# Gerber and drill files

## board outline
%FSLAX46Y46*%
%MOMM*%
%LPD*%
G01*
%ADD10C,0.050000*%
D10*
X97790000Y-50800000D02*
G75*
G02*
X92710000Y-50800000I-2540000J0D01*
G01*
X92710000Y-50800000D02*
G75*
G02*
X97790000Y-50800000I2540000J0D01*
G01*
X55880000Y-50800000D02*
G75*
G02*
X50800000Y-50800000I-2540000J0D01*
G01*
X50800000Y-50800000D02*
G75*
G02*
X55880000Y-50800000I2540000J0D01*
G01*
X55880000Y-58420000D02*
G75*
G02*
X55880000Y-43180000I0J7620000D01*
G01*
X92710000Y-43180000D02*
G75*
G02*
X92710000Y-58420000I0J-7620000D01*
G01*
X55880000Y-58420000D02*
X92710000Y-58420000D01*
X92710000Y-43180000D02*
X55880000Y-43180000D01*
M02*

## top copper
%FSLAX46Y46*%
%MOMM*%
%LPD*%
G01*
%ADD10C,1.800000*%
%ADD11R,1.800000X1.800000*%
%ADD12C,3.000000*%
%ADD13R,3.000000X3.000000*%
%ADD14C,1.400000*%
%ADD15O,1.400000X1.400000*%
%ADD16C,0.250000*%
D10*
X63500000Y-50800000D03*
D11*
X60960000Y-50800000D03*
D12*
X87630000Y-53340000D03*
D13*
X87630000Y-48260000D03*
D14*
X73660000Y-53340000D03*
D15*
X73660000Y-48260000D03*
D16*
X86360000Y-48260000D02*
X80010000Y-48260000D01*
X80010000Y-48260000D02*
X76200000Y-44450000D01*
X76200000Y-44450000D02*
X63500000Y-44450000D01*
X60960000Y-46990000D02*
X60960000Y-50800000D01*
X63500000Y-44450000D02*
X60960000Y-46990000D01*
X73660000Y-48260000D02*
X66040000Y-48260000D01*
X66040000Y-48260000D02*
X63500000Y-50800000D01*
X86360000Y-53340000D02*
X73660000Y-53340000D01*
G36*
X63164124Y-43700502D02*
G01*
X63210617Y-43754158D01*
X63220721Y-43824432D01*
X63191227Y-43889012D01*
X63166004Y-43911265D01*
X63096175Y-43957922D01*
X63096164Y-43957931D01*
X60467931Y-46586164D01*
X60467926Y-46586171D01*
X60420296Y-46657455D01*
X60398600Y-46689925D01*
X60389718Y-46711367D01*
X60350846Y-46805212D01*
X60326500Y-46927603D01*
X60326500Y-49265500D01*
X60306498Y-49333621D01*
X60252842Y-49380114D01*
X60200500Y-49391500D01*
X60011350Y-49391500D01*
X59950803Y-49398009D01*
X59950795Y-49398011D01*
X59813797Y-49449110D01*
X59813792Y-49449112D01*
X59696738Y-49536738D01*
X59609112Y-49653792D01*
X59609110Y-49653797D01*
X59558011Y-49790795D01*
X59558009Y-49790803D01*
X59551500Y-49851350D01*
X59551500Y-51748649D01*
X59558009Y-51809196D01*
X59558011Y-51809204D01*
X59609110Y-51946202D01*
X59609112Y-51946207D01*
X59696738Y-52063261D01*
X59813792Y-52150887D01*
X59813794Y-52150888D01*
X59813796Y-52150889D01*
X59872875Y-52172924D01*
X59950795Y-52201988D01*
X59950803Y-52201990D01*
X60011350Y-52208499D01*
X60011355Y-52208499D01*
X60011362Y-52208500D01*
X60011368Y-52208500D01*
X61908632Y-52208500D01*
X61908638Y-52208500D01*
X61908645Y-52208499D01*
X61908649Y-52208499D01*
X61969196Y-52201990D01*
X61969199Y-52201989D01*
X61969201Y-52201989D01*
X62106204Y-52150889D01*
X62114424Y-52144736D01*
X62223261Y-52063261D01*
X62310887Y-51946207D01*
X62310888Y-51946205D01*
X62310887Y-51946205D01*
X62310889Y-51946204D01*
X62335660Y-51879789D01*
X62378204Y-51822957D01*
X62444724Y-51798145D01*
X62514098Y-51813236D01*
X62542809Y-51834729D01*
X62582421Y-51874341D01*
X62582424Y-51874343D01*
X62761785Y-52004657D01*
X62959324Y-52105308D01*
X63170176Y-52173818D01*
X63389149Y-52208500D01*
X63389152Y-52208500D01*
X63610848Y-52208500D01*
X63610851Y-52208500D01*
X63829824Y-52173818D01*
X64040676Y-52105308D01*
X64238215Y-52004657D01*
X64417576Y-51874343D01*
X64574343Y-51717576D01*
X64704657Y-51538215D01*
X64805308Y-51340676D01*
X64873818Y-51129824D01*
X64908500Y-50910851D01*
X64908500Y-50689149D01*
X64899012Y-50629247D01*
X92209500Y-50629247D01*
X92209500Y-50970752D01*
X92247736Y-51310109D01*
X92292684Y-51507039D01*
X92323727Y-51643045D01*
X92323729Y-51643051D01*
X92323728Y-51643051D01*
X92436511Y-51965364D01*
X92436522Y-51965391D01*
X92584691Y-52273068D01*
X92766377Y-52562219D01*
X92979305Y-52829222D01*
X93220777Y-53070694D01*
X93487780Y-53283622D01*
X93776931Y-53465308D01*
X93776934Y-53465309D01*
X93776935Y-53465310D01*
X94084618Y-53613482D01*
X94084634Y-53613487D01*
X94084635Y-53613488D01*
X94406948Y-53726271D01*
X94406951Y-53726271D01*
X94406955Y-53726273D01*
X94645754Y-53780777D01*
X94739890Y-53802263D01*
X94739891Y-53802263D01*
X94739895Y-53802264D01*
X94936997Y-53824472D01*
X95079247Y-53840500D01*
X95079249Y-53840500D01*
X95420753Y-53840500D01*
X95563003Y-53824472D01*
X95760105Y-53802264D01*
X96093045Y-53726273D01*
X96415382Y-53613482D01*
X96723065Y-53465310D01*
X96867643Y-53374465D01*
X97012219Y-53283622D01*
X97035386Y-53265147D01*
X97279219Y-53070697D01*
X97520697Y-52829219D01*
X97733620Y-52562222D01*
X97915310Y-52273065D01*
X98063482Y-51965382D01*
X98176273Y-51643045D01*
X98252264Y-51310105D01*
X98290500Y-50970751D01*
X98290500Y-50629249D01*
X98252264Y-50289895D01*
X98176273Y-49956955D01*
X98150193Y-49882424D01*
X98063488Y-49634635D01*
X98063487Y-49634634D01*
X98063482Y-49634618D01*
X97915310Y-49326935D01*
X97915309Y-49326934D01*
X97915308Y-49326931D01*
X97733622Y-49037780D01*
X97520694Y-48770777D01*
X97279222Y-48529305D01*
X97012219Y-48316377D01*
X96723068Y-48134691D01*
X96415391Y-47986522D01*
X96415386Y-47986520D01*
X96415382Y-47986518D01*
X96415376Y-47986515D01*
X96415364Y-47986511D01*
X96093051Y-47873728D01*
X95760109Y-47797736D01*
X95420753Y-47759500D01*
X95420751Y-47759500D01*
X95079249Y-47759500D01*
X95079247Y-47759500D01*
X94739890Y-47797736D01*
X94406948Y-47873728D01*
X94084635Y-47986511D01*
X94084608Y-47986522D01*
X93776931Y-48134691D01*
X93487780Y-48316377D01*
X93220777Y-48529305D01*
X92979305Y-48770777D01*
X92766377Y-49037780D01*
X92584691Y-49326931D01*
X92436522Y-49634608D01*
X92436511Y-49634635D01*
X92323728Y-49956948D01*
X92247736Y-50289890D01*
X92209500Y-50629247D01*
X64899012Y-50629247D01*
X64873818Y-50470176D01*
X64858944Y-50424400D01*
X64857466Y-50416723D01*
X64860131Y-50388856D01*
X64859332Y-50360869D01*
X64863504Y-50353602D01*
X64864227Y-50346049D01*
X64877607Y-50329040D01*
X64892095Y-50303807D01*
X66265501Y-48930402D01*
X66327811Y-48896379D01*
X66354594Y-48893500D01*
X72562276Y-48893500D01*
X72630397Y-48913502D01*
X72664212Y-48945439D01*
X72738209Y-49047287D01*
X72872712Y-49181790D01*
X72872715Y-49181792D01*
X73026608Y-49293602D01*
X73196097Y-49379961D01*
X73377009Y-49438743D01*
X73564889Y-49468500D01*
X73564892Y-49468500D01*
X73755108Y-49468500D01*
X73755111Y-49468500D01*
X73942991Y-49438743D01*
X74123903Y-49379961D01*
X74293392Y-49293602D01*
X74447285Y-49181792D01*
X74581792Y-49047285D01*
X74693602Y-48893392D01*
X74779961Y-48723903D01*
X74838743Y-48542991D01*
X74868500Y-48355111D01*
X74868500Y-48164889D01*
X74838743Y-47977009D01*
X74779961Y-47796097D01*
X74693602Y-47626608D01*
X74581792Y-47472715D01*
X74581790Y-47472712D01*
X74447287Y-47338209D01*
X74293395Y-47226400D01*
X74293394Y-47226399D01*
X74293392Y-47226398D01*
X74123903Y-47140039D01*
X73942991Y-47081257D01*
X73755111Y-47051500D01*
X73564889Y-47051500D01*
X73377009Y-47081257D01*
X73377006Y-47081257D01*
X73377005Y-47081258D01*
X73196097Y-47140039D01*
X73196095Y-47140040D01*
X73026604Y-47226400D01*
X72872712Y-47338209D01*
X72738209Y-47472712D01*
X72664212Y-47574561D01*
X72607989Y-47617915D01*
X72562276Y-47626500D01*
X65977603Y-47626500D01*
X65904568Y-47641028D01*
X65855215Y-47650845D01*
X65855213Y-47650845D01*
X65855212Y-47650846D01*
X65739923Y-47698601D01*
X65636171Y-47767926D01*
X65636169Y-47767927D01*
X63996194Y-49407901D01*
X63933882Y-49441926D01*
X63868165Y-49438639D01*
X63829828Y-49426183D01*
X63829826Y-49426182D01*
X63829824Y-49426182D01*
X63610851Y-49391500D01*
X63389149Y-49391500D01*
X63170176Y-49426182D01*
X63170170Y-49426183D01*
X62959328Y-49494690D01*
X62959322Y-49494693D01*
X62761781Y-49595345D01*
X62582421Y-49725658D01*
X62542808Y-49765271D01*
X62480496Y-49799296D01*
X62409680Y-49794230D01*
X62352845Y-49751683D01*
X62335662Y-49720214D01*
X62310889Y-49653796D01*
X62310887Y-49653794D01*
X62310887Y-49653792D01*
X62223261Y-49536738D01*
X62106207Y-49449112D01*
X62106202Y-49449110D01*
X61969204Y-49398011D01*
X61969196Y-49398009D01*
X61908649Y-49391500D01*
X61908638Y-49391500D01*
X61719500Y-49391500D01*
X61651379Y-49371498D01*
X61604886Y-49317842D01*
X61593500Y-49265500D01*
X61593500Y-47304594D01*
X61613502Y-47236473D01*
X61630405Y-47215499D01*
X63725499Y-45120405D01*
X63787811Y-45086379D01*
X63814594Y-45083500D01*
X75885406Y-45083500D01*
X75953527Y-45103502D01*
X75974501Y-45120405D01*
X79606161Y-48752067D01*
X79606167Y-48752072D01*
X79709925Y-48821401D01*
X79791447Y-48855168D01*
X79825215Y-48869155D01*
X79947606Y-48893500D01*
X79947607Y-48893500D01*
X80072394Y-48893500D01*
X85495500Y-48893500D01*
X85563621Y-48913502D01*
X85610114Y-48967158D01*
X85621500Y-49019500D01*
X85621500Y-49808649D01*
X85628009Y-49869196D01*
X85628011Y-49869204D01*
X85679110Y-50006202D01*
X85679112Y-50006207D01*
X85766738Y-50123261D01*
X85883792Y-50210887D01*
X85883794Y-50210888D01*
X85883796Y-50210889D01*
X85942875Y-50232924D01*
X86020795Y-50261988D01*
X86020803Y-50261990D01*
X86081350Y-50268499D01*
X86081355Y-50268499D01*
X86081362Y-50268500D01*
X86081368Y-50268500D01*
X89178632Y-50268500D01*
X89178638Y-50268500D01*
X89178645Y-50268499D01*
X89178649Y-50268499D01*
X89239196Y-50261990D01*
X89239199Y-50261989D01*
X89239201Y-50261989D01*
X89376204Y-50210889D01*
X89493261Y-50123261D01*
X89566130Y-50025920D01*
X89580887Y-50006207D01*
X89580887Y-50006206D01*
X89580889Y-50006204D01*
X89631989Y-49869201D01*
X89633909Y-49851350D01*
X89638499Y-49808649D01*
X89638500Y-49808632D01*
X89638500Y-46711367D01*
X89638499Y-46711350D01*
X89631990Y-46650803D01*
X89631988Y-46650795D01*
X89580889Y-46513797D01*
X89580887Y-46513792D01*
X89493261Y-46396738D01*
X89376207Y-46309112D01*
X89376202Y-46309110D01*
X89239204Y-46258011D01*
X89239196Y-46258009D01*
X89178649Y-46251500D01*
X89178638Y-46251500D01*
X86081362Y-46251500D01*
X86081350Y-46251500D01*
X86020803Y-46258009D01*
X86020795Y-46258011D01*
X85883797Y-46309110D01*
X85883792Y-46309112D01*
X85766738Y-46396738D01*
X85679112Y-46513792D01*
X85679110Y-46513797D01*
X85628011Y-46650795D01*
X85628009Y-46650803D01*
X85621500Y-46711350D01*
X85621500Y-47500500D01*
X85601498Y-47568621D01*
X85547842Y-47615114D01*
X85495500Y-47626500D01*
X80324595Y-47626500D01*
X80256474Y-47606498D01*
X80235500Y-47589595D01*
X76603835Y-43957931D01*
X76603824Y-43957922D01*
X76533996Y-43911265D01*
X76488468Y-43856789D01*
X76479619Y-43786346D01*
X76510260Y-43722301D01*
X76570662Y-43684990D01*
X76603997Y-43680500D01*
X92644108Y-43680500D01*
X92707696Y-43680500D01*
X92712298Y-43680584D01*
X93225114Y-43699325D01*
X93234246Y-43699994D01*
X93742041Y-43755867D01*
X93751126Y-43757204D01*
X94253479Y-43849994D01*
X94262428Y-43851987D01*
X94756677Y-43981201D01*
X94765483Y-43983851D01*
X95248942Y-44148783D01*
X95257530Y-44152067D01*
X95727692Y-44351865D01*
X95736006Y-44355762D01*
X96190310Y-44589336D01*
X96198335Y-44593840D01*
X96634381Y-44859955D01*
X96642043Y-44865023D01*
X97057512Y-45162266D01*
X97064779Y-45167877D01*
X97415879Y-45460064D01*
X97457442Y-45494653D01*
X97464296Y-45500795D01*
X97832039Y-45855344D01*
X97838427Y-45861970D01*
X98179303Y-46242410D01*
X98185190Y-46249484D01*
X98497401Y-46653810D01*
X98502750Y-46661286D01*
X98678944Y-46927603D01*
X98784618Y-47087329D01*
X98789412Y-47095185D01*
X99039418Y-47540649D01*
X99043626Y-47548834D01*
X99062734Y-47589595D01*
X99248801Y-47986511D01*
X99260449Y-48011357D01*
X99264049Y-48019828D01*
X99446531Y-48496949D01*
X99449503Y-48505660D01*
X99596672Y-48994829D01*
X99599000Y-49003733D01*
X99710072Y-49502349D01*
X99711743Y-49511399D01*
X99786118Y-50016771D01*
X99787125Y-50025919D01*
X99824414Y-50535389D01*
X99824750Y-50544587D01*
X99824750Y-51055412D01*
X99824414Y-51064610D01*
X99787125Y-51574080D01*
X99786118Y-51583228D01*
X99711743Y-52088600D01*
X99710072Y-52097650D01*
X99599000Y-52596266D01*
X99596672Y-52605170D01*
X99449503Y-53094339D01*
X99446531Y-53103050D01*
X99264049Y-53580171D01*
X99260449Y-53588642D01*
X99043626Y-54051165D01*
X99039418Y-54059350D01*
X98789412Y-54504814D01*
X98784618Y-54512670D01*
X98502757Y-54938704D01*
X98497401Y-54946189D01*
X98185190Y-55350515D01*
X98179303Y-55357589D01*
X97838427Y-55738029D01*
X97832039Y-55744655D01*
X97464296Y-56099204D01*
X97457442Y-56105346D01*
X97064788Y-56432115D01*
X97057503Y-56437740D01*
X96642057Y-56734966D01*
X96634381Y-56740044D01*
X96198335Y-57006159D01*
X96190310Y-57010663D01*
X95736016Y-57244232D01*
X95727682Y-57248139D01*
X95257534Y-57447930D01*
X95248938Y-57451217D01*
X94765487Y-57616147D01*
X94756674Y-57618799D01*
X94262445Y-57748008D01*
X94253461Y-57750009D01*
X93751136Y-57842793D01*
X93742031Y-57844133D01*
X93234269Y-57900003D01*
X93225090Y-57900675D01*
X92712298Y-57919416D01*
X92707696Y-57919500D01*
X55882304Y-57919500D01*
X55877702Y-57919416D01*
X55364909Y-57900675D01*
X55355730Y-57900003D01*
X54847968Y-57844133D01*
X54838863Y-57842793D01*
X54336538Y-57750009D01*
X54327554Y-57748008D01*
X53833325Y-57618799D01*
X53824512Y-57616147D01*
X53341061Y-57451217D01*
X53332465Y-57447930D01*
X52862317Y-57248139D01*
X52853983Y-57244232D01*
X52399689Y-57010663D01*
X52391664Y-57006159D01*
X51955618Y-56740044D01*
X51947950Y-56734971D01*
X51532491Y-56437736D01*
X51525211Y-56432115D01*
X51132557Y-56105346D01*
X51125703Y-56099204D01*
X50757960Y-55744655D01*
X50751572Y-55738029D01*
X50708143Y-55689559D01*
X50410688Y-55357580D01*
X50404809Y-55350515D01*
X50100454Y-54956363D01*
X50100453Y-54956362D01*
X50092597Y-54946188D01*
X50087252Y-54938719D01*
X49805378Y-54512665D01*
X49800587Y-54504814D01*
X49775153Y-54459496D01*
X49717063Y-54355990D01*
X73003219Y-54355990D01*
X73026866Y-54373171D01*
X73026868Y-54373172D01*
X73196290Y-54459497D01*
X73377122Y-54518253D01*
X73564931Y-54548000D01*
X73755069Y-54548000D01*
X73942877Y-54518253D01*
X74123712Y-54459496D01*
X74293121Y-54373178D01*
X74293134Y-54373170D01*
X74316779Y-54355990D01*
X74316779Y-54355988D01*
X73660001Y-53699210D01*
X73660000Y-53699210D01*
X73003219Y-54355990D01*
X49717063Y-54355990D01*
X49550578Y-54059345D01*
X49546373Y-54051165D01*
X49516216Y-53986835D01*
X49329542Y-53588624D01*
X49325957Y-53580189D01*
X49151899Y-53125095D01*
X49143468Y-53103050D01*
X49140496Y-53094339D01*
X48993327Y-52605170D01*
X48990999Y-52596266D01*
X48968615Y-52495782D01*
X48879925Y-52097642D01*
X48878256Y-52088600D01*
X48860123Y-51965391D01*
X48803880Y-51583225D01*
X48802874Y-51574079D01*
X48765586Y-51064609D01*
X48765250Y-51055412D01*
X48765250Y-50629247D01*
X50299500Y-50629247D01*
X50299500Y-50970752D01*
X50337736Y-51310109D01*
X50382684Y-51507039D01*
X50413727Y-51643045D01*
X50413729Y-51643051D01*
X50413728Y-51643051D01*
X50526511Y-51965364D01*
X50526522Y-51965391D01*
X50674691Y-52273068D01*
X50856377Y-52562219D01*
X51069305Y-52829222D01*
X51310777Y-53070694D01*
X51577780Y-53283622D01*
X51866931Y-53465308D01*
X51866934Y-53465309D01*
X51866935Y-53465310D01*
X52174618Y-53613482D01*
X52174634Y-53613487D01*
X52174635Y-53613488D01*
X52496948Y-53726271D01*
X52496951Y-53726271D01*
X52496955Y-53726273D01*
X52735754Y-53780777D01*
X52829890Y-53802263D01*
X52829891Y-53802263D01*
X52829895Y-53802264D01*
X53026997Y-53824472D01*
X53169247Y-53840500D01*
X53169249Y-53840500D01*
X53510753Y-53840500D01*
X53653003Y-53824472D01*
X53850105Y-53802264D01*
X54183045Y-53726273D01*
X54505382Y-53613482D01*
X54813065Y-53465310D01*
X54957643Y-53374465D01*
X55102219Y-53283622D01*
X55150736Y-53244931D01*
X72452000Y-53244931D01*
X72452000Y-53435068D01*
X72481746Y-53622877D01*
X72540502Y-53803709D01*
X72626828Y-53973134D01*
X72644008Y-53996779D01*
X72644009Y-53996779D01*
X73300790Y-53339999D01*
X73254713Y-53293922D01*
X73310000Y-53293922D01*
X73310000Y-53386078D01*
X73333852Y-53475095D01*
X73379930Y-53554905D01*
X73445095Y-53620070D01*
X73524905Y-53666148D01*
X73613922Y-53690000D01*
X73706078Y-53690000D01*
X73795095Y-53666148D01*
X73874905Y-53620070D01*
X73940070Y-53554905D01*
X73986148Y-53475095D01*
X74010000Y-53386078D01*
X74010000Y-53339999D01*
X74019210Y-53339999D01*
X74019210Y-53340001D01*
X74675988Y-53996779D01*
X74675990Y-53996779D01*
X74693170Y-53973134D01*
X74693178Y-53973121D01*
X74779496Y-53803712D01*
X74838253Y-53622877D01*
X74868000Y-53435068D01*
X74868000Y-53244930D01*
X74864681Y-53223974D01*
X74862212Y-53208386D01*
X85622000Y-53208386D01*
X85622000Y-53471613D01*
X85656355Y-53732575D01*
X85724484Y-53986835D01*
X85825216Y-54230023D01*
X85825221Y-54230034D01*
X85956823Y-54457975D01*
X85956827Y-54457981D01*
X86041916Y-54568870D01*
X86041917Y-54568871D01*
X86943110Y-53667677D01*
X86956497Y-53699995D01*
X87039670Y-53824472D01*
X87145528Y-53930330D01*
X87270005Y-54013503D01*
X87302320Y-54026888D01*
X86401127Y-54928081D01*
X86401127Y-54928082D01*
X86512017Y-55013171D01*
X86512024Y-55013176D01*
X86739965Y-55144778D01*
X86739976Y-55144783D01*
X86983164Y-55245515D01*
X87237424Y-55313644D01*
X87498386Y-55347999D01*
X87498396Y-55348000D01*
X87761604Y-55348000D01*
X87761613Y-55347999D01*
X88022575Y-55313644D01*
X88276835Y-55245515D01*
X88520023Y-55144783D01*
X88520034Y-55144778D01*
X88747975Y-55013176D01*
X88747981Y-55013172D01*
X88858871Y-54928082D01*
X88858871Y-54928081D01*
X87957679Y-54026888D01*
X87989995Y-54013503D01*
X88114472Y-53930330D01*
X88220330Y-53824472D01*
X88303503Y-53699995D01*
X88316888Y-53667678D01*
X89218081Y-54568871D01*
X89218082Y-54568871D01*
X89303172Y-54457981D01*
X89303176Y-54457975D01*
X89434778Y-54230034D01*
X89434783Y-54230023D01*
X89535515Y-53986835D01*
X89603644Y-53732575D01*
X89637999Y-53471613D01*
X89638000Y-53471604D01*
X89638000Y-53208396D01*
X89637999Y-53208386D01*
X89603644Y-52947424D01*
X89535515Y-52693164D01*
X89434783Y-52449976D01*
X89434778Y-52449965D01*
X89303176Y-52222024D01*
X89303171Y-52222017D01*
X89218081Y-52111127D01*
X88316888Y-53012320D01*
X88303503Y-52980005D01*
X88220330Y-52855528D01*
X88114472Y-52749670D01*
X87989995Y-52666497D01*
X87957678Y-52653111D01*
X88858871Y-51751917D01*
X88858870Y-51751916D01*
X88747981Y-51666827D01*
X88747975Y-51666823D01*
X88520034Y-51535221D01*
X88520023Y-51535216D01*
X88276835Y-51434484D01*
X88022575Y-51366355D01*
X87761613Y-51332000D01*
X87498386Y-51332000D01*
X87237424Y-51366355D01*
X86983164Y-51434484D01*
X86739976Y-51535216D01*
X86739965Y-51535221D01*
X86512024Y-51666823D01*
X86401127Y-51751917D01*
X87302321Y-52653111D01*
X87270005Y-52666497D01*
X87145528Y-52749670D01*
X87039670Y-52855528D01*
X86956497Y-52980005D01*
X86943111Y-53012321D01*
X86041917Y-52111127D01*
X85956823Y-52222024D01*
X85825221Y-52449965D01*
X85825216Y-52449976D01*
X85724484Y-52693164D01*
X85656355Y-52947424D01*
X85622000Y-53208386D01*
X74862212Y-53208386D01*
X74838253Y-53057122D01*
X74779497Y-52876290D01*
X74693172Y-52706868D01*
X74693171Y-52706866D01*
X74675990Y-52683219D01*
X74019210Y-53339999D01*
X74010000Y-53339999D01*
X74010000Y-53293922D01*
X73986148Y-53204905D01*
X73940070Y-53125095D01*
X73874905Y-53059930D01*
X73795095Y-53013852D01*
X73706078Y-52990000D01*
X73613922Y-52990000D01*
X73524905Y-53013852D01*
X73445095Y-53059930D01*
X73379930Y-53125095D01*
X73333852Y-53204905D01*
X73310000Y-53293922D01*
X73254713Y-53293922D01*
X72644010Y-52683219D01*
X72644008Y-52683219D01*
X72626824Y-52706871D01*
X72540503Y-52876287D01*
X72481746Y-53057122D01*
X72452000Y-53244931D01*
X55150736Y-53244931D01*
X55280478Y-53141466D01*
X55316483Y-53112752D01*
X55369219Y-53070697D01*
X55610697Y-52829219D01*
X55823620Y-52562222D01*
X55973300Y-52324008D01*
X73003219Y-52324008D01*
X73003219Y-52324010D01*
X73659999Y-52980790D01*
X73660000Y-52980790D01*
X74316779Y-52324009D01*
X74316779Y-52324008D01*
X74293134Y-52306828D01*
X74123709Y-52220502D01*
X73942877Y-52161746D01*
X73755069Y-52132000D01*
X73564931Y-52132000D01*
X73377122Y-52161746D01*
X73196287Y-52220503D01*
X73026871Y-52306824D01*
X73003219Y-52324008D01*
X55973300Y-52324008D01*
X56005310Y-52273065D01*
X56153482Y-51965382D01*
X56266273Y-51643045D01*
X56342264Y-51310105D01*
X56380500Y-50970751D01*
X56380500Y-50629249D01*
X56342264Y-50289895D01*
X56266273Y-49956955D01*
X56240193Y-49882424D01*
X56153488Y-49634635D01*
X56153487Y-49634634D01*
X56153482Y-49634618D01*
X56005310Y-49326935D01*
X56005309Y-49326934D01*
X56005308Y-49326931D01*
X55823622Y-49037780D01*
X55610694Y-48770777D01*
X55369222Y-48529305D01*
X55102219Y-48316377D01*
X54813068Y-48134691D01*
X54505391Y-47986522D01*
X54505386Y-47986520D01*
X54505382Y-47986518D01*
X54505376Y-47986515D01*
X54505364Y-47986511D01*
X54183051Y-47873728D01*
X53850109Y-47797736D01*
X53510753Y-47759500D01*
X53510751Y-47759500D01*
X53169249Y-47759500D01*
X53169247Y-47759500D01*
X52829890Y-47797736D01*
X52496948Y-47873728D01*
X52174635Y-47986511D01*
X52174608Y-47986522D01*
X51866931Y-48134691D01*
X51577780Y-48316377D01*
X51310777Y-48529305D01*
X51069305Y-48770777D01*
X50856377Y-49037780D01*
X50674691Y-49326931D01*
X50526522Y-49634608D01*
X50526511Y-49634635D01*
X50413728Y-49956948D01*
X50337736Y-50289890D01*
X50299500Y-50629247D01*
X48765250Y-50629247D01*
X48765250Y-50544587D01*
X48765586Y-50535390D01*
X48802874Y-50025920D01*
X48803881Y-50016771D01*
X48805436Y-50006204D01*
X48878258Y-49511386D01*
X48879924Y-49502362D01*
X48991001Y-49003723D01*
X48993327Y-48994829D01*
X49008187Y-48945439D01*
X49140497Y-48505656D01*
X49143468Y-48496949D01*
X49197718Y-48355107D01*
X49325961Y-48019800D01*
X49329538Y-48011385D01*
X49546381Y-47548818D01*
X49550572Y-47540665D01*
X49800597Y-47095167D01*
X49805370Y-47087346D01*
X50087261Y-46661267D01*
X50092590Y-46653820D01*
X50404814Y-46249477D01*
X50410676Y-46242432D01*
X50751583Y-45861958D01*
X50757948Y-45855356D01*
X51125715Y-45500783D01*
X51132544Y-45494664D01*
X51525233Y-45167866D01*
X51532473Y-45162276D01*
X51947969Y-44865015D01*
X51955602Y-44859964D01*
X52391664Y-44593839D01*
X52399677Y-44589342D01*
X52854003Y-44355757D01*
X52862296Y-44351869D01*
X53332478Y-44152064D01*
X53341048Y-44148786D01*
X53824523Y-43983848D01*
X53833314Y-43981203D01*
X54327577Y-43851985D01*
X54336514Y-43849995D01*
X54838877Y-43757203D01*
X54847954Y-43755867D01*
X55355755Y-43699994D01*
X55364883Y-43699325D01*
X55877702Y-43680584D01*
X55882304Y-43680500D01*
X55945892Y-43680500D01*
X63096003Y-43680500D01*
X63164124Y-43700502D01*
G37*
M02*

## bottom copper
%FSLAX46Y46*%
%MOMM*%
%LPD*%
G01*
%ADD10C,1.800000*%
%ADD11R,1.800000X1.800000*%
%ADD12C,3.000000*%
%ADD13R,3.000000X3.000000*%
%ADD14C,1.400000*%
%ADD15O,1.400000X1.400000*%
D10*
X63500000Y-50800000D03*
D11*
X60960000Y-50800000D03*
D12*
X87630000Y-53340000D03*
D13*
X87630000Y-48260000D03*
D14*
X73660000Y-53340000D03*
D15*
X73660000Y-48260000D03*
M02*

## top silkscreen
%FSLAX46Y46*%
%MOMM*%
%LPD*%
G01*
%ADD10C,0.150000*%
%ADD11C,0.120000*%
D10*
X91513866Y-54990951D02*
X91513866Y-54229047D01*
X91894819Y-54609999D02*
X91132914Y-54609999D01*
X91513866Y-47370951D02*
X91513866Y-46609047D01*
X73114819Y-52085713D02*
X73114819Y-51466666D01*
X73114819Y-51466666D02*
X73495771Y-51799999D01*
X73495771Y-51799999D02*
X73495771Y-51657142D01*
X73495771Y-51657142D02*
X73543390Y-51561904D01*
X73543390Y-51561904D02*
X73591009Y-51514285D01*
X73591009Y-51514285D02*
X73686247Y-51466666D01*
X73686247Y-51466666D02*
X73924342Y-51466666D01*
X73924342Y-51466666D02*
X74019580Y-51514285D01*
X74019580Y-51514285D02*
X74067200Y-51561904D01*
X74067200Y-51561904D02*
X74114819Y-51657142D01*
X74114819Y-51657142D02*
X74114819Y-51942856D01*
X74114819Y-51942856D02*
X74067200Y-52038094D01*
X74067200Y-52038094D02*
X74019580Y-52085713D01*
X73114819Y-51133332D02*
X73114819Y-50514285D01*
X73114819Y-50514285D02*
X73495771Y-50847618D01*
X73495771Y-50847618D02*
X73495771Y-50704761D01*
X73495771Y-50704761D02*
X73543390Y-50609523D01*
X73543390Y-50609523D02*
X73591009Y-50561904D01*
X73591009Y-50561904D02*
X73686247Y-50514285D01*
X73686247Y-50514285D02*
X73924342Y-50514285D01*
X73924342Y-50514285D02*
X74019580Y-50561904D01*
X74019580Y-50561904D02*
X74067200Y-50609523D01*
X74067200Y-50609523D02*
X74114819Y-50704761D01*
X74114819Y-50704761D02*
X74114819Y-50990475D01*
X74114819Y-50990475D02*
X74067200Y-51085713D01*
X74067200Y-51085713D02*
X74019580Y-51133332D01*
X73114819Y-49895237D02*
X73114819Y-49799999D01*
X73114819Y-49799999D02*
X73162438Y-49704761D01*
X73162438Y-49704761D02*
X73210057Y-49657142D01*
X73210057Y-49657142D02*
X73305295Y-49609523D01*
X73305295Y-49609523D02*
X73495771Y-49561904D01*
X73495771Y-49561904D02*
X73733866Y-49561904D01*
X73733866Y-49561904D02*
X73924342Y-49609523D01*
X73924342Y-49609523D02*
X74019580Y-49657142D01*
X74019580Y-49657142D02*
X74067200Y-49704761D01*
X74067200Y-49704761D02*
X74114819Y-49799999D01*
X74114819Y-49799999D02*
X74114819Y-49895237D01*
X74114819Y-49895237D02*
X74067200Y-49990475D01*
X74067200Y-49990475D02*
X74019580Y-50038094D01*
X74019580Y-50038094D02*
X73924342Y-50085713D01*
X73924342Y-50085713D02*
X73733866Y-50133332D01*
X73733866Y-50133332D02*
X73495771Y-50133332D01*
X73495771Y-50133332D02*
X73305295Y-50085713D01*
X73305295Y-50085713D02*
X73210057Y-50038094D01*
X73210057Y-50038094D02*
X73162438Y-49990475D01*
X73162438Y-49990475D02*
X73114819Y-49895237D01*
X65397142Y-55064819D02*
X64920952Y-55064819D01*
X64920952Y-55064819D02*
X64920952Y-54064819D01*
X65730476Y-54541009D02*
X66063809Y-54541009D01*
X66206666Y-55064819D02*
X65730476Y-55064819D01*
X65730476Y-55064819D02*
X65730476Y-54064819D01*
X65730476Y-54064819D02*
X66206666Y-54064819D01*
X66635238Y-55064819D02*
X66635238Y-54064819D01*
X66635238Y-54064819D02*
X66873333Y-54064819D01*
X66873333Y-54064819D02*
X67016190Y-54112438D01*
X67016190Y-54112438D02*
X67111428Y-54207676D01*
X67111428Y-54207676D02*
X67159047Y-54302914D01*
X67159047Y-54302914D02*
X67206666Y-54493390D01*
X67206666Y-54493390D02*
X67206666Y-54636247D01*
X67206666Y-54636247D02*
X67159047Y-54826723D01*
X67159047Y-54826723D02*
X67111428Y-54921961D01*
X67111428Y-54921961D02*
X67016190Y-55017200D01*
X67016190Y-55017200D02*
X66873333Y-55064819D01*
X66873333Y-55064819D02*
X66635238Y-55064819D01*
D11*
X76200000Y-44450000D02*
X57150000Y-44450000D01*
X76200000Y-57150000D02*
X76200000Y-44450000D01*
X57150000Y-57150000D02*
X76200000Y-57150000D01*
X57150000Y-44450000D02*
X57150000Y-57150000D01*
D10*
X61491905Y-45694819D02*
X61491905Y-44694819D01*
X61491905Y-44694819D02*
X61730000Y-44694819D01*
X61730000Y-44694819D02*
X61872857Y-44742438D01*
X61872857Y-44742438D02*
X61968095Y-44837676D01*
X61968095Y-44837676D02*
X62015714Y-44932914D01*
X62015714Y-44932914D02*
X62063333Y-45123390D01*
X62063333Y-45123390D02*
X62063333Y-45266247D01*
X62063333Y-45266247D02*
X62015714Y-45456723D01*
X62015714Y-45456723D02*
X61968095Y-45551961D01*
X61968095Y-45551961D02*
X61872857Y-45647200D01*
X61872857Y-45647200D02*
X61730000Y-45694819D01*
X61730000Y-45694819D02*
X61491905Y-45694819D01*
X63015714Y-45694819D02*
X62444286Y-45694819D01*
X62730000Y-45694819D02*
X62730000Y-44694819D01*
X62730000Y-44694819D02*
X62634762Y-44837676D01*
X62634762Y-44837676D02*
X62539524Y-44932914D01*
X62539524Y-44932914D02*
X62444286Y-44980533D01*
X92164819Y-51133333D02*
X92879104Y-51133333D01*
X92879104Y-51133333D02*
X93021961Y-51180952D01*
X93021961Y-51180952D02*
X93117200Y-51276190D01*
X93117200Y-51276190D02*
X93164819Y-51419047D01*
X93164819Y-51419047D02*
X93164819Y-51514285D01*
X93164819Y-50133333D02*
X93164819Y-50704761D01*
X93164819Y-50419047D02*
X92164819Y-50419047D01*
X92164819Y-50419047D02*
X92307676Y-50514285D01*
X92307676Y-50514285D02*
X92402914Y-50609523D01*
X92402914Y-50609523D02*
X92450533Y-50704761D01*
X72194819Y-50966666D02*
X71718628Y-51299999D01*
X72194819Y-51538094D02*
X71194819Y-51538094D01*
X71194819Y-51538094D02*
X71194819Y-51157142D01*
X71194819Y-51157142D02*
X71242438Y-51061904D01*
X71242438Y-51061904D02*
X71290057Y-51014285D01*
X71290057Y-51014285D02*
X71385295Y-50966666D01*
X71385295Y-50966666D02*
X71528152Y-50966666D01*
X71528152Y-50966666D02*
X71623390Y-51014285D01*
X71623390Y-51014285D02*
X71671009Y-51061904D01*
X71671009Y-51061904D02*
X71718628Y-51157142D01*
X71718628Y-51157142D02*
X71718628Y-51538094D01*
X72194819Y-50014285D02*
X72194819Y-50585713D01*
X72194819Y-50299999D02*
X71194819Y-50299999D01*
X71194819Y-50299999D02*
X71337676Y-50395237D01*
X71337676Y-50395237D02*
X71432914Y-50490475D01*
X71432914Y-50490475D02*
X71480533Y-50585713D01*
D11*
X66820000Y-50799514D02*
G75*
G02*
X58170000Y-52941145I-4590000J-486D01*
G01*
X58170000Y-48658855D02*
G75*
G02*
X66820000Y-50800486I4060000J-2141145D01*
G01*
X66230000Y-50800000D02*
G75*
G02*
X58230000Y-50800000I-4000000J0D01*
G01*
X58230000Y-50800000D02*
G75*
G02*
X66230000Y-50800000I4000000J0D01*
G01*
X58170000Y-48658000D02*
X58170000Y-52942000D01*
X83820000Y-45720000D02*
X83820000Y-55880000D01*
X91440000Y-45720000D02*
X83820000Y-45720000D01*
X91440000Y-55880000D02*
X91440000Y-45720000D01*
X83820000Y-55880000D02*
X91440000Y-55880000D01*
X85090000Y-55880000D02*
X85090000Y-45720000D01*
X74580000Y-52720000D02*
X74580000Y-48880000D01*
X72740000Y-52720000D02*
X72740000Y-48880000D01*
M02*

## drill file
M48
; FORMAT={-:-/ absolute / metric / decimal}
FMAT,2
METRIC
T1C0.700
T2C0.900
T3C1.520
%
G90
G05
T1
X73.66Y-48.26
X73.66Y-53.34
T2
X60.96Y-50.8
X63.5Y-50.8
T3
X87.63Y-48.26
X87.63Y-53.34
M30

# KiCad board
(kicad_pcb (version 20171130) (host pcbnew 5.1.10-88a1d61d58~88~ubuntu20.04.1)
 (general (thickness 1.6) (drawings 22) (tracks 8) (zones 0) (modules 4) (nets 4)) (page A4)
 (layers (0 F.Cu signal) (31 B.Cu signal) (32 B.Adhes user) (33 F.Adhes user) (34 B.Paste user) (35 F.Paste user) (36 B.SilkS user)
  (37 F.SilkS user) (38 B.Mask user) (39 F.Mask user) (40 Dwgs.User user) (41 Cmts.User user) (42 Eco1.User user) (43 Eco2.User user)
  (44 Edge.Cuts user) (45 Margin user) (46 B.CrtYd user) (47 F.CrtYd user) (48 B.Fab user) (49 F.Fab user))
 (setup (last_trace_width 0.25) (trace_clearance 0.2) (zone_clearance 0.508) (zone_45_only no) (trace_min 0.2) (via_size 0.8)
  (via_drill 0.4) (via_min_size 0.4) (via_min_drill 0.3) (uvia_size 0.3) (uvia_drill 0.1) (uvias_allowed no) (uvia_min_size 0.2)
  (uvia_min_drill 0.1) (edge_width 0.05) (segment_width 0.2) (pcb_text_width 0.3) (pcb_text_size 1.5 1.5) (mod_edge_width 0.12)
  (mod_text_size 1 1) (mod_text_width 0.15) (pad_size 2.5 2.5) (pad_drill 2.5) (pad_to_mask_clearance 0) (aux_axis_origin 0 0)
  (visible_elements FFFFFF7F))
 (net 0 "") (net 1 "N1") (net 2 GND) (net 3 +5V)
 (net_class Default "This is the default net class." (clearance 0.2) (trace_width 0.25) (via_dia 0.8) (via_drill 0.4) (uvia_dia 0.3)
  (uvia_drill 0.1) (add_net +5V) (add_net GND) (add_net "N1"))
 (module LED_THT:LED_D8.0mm (layer F.Cu) (at 60.96 50.8)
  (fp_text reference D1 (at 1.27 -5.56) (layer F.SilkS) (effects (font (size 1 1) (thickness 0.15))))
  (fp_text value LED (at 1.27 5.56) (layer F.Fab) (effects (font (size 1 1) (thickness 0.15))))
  (fp_arc (start 1.27 0) (end -2.79 2.141145) (angle -152.2) (layer F.SilkS) (width 0.12))
  (fp_arc (start 1.27 0) (end -2.79 -2.141145) (angle 152.2) (layer F.SilkS) (width 0.12))
  (fp_circle (center 1.27 0) (end 5.27 0) (layer F.SilkS) (width 0.12))
  (fp_line (start -2.79 -2.142) (end -2.79 2.142) (layer F.SilkS) (width 0.12))
  (pad 2 thru_hole circle (at 2.54 0) (size 1.8 1.8) (drill 0.9) (layers *.Cu *.Mask) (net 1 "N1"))
  (pad 1 thru_hole rect (at 0 0) (size 1.8 1.8) (drill 0.9) (layers *.Cu *.Mask) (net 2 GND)))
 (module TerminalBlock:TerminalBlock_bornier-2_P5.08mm (layer F.Cu) (at 87.63 48.26 270)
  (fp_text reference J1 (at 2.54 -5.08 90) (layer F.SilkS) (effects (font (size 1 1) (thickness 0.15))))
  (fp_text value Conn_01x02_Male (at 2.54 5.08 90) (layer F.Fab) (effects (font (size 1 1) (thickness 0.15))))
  (fp_line (start -2.54 3.81) (end 7.62 3.81) (layer F.SilkS) (width 0.12))
  (fp_line (start -2.54 -3.81) (end -2.54 3.81) (layer F.SilkS) (width 0.12))
  (fp_line (start 7.62 -3.81) (end -2.54 -3.81) (layer F.SilkS) (width 0.12))
  (fp_line (start 7.62 3.81) (end 7.62 -3.81) (layer F.SilkS) (width 0.12))
  (fp_line (start 7.62 2.54) (end -2.54 2.54) (layer F.SilkS) (width 0.12))
  (pad 2 thru_hole circle (at 5.08 0 270) (size 3 3) (drill 1.52) (layers *.Cu *.Mask) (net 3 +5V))
  (pad 1 thru_hole rect (at 0 0 270) (size 3 3) (drill 1.52) (layers *.Cu *.Mask) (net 2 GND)))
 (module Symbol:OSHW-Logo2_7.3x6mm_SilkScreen (layer B.Cu) (at 80.01 53.34 180)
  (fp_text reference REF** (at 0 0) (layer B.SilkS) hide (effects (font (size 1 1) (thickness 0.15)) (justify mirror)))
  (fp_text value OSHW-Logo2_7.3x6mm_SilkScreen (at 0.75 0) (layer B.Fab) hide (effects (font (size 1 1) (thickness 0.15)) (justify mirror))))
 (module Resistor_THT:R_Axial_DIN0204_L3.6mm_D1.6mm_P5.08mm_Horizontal (layer F.Cu) (at 73.66 53.34 90)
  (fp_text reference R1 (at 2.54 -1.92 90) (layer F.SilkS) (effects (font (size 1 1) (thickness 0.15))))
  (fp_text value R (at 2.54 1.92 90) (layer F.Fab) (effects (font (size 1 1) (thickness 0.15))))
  (fp_line (start 0.62 0.92) (end 4.46 0.92) (layer F.SilkS) (width 0.12))
  (fp_line (start 0.62 -0.92) (end 4.46 -0.92) (layer F.SilkS) (width 0.12))
  (pad 1 thru_hole circle (at 0 0 90) (size 1.4 1.4) (drill 0.7) (layers *.Cu *.Mask) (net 3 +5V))
  (pad 2 thru_hole oval (at 5.08 0 90) (size 1.4 1.4) (drill 0.7) (layers *.Cu *.Mask) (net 1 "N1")))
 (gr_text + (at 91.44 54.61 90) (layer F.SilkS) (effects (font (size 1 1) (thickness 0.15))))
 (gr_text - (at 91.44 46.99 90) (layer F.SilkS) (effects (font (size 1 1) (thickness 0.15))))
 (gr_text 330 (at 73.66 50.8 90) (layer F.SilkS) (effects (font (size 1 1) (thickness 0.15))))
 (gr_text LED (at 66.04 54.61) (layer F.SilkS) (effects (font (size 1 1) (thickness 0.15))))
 (gr_line (start 76.2 44.45) (end 57.15 44.45) (layer F.SilkS) (width 0.12))
 (gr_line (start 76.2 57.15) (end 76.2 44.45) (layer F.SilkS) (width 0.12))
 (gr_line (start 57.15 57.15) (end 76.2 57.15) (layer F.SilkS) (width 0.12))
 (gr_line (start 57.15 44.45) (end 57.15 57.15) (layer F.SilkS) (width 0.12))
 (gr_circle (center 95.25 50.8) (end 95.25 53.34) (layer Edge.Cuts) (width 0.05))
 (gr_circle (center 53.34 50.8) (end 55.88 50.8) (layer Edge.Cuts) (width 0.05))
 (gr_arc (start 55.88 50.8) (end 55.88 43.18) (angle -180) (layer Edge.Cuts) (width 0.05))
 (gr_arc (start 92.71 50.8) (end 92.71 58.42) (angle -180) (layer Edge.Cuts) (width 0.05))
 (gr_line (start 55.88 58.42) (end 92.71 58.42) (layer Edge.Cuts) (width 0.05))
 (gr_line (start 92.71 43.18) (end 55.88 43.18) (layer Edge.Cuts) (width 0.05))
 (segment (start 86.36 48.26) (end 80.01 48.26) (width 0.25) (layer F.Cu) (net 2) (status 10))
 (segment (start 80.01 48.26) (end 76.2 44.45) (width 0.25) (layer F.Cu) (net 2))
 (segment (start 76.2 44.45) (end 63.5 44.45) (width 0.25) (layer F.Cu) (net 2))
 (segment (start 60.96 46.99) (end 60.96 50.8) (width 0.25) (layer F.Cu) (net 2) (status 20))
 (segment (start 63.5 44.45) (end 60.96 46.99) (width 0.25) (layer F.Cu) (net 2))
 (segment (start 73.66 48.26) (end 66.04 48.26) (width 0.25) (layer F.Cu) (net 1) (status 10))
 (segment (start 66.04 48.26) (end 63.5 50.8) (width 0.25) (layer F.Cu) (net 1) (status 20))
 (segment (start 86.36 53.34) (end 73.66 53.34) (width 0.25) (layer F.Cu) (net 3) (status 30))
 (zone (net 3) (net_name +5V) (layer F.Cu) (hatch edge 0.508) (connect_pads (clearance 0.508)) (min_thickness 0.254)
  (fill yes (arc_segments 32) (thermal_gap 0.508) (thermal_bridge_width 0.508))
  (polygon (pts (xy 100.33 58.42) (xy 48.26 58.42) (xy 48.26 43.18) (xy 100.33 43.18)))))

